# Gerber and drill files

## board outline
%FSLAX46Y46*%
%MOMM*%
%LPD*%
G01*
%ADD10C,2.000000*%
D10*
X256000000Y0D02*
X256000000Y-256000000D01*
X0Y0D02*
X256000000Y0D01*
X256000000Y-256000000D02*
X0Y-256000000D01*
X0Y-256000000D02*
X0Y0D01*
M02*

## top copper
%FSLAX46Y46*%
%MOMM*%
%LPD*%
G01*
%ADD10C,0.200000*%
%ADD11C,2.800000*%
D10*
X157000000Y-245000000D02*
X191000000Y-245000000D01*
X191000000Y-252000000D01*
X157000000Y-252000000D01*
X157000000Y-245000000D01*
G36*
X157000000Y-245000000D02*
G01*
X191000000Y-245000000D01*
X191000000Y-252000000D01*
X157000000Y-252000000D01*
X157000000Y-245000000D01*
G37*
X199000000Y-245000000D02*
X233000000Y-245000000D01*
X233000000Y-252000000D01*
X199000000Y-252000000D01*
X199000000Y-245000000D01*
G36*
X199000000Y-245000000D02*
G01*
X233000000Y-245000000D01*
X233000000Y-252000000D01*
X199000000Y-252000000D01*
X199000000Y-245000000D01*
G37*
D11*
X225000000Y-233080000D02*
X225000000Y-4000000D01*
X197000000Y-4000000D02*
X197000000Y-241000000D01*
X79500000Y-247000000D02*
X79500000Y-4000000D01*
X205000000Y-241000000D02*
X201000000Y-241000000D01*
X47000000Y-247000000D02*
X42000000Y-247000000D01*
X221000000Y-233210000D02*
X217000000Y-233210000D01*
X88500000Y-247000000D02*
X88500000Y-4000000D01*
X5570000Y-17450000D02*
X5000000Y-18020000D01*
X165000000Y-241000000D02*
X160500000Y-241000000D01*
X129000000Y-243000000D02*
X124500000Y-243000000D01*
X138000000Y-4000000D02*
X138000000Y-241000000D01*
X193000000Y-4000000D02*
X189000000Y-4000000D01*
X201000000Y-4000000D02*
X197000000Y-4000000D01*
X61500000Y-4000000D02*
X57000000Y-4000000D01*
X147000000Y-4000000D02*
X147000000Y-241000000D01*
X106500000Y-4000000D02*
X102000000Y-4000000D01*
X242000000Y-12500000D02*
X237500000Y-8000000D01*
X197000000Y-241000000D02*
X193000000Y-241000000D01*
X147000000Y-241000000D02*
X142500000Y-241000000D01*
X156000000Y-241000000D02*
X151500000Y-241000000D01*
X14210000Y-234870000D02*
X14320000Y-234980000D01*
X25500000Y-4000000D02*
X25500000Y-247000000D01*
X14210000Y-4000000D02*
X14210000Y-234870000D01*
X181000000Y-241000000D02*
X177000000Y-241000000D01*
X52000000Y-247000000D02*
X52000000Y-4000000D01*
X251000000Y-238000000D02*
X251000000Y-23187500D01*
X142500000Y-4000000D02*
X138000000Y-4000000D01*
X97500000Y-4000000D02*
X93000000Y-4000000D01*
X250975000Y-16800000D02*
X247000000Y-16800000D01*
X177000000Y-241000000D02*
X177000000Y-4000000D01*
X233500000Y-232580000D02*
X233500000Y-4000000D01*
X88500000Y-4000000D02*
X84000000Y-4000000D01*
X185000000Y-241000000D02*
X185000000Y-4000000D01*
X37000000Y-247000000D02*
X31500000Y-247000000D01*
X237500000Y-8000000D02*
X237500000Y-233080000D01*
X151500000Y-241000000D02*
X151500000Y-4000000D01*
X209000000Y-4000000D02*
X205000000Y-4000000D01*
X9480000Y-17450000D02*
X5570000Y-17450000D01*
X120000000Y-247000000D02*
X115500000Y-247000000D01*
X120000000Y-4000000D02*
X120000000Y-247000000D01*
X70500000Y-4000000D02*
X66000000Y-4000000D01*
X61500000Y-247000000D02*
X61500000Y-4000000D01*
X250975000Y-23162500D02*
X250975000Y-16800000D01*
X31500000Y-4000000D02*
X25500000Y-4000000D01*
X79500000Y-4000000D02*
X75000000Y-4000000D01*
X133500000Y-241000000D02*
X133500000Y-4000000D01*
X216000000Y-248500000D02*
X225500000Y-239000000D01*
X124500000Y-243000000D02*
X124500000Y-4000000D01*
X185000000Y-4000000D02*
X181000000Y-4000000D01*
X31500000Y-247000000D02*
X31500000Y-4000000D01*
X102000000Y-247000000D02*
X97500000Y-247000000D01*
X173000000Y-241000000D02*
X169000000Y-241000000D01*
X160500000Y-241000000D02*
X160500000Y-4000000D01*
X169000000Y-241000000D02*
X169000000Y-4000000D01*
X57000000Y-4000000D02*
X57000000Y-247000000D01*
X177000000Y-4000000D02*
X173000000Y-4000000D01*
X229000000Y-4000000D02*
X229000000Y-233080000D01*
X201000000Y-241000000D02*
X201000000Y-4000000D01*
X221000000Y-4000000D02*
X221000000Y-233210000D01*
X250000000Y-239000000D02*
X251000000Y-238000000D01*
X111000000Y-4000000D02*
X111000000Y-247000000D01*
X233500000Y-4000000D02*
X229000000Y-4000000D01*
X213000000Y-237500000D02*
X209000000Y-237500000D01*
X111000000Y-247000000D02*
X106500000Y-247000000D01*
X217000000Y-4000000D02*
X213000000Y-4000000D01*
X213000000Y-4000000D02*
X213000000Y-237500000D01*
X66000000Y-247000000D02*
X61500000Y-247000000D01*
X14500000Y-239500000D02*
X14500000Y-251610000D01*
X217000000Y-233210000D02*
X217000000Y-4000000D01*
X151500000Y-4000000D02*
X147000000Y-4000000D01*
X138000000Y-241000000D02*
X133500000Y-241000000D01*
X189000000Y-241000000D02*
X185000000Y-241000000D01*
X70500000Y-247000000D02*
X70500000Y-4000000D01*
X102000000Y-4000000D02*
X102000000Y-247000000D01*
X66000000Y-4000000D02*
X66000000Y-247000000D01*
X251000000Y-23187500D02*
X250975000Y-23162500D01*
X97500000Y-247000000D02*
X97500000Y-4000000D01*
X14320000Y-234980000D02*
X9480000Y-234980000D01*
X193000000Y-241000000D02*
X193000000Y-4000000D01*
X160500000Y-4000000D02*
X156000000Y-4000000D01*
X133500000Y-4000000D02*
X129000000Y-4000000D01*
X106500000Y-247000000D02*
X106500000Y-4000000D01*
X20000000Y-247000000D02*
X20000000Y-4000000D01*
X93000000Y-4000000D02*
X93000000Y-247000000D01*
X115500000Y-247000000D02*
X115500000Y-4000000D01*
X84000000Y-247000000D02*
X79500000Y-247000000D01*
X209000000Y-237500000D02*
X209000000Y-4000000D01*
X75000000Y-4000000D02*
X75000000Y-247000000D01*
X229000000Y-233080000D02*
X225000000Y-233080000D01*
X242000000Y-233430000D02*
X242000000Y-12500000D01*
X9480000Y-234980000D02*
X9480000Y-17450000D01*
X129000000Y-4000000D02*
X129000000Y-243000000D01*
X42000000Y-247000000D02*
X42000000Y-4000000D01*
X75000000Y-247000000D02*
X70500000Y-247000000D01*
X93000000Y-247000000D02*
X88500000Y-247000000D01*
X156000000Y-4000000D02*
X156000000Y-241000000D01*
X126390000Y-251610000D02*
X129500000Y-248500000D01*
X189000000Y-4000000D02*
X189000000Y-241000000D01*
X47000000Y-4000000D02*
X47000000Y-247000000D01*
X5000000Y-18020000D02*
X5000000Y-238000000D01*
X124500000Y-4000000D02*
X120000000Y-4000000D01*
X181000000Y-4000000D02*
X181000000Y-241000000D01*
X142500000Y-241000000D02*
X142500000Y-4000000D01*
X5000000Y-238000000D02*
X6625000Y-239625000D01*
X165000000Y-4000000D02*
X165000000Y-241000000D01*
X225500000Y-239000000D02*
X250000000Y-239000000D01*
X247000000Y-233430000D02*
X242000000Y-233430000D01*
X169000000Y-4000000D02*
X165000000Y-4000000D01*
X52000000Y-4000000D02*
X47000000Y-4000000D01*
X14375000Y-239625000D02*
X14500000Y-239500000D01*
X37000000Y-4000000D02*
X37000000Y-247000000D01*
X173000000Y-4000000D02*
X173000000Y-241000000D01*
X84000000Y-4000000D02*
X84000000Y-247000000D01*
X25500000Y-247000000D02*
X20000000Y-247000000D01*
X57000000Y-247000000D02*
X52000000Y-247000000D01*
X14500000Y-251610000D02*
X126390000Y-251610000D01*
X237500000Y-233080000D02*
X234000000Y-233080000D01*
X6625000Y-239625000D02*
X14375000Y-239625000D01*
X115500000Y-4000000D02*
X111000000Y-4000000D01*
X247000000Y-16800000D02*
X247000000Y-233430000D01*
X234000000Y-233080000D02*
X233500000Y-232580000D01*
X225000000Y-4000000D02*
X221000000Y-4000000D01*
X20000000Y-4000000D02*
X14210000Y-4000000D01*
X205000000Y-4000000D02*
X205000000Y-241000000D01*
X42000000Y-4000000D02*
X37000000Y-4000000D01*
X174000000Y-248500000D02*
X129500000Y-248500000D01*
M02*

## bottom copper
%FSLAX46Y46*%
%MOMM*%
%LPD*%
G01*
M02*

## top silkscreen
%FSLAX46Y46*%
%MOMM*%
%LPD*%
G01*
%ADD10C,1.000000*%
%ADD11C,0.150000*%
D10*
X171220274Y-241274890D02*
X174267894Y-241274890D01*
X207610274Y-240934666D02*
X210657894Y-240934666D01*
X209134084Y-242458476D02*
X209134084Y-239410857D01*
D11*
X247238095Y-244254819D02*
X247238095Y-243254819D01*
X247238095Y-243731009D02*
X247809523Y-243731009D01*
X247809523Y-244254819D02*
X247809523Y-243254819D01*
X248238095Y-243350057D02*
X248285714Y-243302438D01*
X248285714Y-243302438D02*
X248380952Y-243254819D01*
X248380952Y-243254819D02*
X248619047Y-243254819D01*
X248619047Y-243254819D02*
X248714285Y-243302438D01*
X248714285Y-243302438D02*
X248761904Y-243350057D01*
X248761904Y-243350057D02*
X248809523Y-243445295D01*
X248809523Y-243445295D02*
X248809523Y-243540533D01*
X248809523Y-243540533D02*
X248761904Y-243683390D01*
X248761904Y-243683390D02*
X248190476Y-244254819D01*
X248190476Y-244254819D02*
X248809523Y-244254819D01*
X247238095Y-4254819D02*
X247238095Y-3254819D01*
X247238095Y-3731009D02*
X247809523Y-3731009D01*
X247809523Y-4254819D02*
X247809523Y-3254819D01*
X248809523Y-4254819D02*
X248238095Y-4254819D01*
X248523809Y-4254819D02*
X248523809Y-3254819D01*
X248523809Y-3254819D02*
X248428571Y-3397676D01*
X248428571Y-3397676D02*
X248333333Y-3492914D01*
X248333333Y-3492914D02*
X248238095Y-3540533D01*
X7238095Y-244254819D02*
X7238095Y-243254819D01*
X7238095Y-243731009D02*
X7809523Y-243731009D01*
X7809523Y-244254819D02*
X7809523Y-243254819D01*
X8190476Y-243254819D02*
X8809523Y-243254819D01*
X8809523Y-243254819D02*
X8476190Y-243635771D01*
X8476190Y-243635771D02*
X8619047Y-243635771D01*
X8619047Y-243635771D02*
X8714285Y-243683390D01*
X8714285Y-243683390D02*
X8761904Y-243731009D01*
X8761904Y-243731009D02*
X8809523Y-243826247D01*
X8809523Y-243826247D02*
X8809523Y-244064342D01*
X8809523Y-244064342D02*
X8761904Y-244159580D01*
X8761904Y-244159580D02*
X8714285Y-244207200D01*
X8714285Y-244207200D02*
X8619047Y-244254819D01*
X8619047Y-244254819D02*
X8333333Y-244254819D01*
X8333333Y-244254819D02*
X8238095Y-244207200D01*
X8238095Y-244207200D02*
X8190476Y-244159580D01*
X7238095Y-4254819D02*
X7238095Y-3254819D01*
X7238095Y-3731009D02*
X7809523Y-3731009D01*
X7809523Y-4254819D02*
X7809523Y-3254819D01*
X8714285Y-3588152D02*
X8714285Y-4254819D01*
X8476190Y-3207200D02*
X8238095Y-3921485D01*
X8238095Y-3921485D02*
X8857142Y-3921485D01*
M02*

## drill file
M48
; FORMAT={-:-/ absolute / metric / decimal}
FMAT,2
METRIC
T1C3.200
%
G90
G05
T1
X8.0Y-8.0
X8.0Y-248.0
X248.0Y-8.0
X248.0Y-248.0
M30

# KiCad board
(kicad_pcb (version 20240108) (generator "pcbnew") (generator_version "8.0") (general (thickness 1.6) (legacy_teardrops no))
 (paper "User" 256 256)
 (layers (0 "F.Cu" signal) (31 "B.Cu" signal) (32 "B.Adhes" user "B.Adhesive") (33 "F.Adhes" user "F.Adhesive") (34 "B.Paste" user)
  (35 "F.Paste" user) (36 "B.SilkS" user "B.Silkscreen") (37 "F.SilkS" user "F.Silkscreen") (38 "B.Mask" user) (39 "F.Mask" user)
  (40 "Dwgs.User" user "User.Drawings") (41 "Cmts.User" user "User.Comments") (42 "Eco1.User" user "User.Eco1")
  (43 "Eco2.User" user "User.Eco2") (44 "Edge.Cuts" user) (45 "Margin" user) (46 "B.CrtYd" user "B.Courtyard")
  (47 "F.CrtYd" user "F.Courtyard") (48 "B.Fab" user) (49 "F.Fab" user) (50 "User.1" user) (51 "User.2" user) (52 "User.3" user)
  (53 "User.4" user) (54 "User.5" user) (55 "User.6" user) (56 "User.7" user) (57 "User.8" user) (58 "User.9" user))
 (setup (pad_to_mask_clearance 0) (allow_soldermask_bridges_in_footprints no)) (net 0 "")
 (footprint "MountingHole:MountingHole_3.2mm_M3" (layer "F.Cu") (at 248 248)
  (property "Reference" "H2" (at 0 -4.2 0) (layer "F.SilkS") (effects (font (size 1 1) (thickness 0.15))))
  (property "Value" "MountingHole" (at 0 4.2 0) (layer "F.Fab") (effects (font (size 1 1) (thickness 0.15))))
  (pad "" np_thru_hole circle (at 0 0) (size 3.2 3.2) (drill 3.2) (layers "*.Cu" "*.Mask")))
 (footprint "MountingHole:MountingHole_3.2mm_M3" (layer "F.Cu") (at 248 8)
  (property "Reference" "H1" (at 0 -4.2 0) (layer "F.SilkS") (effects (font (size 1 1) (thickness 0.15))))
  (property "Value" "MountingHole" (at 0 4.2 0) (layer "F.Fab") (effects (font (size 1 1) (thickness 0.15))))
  (pad "" np_thru_hole circle (at 0 0) (size 3.2 3.2) (drill 3.2) (layers "*.Cu" "*.Mask")))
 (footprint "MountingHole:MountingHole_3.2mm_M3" (layer "F.Cu") (at 8 248)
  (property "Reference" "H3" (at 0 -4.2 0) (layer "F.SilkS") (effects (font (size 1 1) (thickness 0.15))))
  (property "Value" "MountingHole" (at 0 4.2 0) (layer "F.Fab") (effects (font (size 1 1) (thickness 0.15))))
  (pad "" np_thru_hole circle (at 0 0) (size 3.2 3.2) (drill 3.2) (layers "*.Cu" "*.Mask")))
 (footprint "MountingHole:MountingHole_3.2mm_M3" (layer "F.Cu") (at 8 8)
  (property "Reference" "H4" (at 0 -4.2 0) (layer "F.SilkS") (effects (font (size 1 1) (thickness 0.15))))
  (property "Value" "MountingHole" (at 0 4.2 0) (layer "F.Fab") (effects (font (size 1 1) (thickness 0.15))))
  (pad "" np_thru_hole circle (at 0 0) (size 3.2 3.2) (drill 3.2) (layers "*.Cu" "*.Mask")))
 (gr_rect (start 157 245) (end 191 252) (stroke (width 0.2) (type solid)) (fill solid) (layer "F.Cu"))
 (gr_rect (start 199 245) (end 233 252) (stroke (width 0.2) (type solid)) (fill solid) (layer "F.Cu"))
 (gr_line (start 256 0) (end 256 256) (stroke (width 2) (type default)) (layer "Edge.Cuts"))
 (gr_line (start 0 0) (end 256 0) (stroke (width 2) (type default)) (layer "Edge.Cuts"))
 (gr_line (start 256 256) (end 0 256) (stroke (width 2) (type default)) (layer "Edge.Cuts"))
 (gr_line (start 0 256) (end 0 0) (stroke (width 2) (type default)) (layer "Edge.Cuts"))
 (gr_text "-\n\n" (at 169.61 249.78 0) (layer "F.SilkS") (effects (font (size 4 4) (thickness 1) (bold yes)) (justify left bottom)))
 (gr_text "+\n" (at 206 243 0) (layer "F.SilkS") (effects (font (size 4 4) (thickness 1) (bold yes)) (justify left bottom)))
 (segment (start 225 233.08) (end 225 4) (width 2.8) (layer "F.Cu") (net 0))
 (segment (start 197 4) (end 197 241) (width 2.8) (layer "F.Cu") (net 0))
 (segment (start 79.5 247) (end 79.5 4) (width 2.8) (layer "F.Cu") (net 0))
 (segment (start 205 241) (end 201 241) (width 2.8) (layer "F.Cu") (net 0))
 (segment (start 47 247) (end 42 247) (width 2.8) (layer "F.Cu") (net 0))
 (segment (start 221 233.21) (end 217 233.21) (width 2.8) (layer "F.Cu") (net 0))
 (segment (start 88.5 247) (end 88.5 4) (width 2.8) (layer "F.Cu") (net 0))
 (segment (start 5.57 17.45) (end 5 18.02) (width 2.8) (layer "F.Cu") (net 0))
 (segment (start 165 241) (end 160.5 241) (width 2.8) (layer "F.Cu") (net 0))
 (segment (start 129 243) (end 124.5 243) (width 2.8) (layer "F.Cu") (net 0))
 (segment (start 138 4) (end 138 241) (width 2.8) (layer "F.Cu") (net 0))
 (segment (start 193 4) (end 189 4) (width 2.8) (layer "F.Cu") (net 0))
 (segment (start 201 4) (end 197 4) (width 2.8) (layer "F.Cu") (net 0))
 (segment (start 61.5 4) (end 57 4) (width 2.8) (layer "F.Cu") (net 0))
 (segment (start 147 4) (end 147 241) (width 2.8) (layer "F.Cu") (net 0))
 (segment (start 106.5 4) (end 102 4) (width 2.8) (layer "F.Cu") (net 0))
 (segment (start 242 12.5) (end 237.5 8) (width 2.8) (layer "F.Cu") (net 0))
 (segment (start 197 241) (end 193 241) (width 2.8) (layer "F.Cu") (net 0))
 (segment (start 147 241) (end 142.5 241) (width 2.8) (layer "F.Cu") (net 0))
 (segment (start 156 241) (end 151.5 241) (width 2.8) (layer "F.Cu") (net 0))
 (segment (start 14.21 234.87) (end 14.32 234.98) (width 2.8) (layer "F.Cu") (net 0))
 (segment (start 25.5 4) (end 25.5 247) (width 2.8) (layer "F.Cu") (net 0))
 (segment (start 14.21 4) (end 14.21 234.87) (width 2.8) (layer "F.Cu") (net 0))
 (segment (start 181 241) (end 177 241) (width 2.8) (layer "F.Cu") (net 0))
 (segment (start 52 247) (end 52 4) (width 2.8) (layer "F.Cu") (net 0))
 (segment (start 251 238) (end 251 23.1875) (width 2.8) (layer "F.Cu") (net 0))
 (segment (start 142.5 4) (end 138 4) (width 2.8) (layer "F.Cu") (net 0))
 (segment (start 97.5 4) (end 93 4) (width 2.8) (layer "F.Cu") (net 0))
 (segment (start 250.975 16.8) (end 247 16.8) (width 2.8) (layer "F.Cu") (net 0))
 (segment (start 177 241) (end 177 4) (width 2.8) (layer "F.Cu") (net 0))
 (segment (start 233.5 232.58) (end 233.5 4) (width 2.8) (layer "F.Cu") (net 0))
 (segment (start 88.5 4) (end 84 4) (width 2.8) (layer "F.Cu") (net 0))
 (segment (start 185 241) (end 185 4) (width 2.8) (layer "F.Cu") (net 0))
 (segment (start 37 247) (end 31.5 247) (width 2.8) (layer "F.Cu") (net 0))
 (segment (start 237.5 8) (end 237.5 233.08) (width 2.8) (layer "F.Cu") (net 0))
 (segment (start 151.5 241) (end 151.5 4) (width 2.8) (layer "F.Cu") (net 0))
 (segment (start 209 4) (end 205 4) (width 2.8) (layer "F.Cu") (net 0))
 (segment (start 9.48 17.45) (end 5.57 17.45) (width 2.8) (layer "F.Cu") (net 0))
 (segment (start 120 247) (end 115.5 247) (width 2.8) (layer "F.Cu") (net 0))
 (segment (start 120 4) (end 120 247) (width 2.8) (layer "F.Cu") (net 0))
 (segment (start 70.5 4) (end 66 4) (width 2.8) (layer "F.Cu") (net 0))
 (segment (start 61.5 247) (end 61.5 4) (width 2.8) (layer "F.Cu") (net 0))
 (segment (start 250.975 23.1625) (end 250.975 16.8) (width 2.8) (layer "F.Cu") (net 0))
 (segment (start 31.5 4) (end 25.5 4) (width 2.8) (layer "F.Cu") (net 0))
 (segment (start 79.5 4) (end 75 4) (width 2.8) (layer "F.Cu") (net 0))
 (segment (start 133.5 241) (end 133.5 4) (width 2.8) (layer "F.Cu") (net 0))
 (segment (start 216 248.5) (end 225.5 239) (width 2.8) (layer "F.Cu") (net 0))
 (segment (start 124.5 243) (end 124.5 4) (width 2.8) (layer "F.Cu") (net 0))
 (segment (start 185 4) (end 181 4) (width 2.8) (layer "F.Cu") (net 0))
 (segment (start 31.5 247) (end 31.5 4) (width 2.8) (layer "F.Cu") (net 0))
 (segment (start 102 247) (end 97.5 247) (width 2.8) (layer "F.Cu") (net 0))
 (segment (start 173 241) (end 169 241) (width 2.8) (layer "F.Cu") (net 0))
 (segment (start 160.5 241) (end 160.5 4) (width 2.8) (layer "F.Cu") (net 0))
 (segment (start 169 241) (end 169 4) (width 2.8) (layer "F.Cu") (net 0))
 (segment (start 57 4) (end 57 247) (width 2.8) (layer "F.Cu") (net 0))
 (segment (start 177 4) (end 173 4) (width 2.8) (layer "F.Cu") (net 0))
 (segment (start 229 4) (end 229 233.08) (width 2.8) (layer "F.Cu") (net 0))
 (segment (start 201 241) (end 201 4) (width 2.8) (layer "F.Cu") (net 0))
 (segment (start 221 4) (end 221 233.21) (width 2.8) (layer "F.Cu") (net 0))
 (segment (start 250 239) (end 251 238) (width 2.8) (layer "F.Cu") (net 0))
 (segment (start 111 4) (end 111 247) (width 2.8) (layer "F.Cu") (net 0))
 (segment (start 233.5 4) (end 229 4) (width 2.8) (layer "F.Cu") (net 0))
 (segment (start 213 237.5) (end 209 237.5) (width 2.8) (layer "F.Cu") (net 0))
 (segment (start 111 247) (end 106.5 247) (width 2.8) (layer "F.Cu") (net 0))
 (segment (start 217 4) (end 213 4) (width 2.8) (layer "F.Cu") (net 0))
 (segment (start 213 4) (end 213 237.5) (width 2.8) (layer "F.Cu") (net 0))
 (segment (start 66 247) (end 61.5 247) (width 2.8) (layer "F.Cu") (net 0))
 (segment (start 14.5 239.5) (end 14.5 251.61) (width 2.8) (layer "F.Cu") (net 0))
 (segment (start 217 233.21) (end 217 4) (width 2.8) (layer "F.Cu") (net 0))
 (segment (start 151.5 4) (end 147 4) (width 2.8) (layer "F.Cu") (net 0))
 (segment (start 138 241) (end 133.5 241) (width 2.8) (layer "F.Cu") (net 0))
 (segment (start 189 241) (end 185 241) (width 2.8) (layer "F.Cu") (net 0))
 (segment (start 70.5 247) (end 70.5 4) (width 2.8) (layer "F.Cu") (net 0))
 (segment (start 102 4) (end 102 247) (width 2.8) (layer "F.Cu") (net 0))
 (segment (start 66 4) (end 66 247) (width 2.8) (layer "F.Cu") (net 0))
 (segment (start 251 23.1875) (end 250.975 23.1625) (width 2.8) (layer "F.Cu") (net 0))
 (segment (start 97.5 247) (end 97.5 4) (width 2.8) (layer "F.Cu") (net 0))
 (segment (start 14.32 234.98) (end 9.48 234.98) (width 2.8) (layer "F.Cu") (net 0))
 (segment (start 193 241) (end 193 4) (width 2.8) (layer "F.Cu") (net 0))
 (segment (start 160.5 4) (end 156 4) (width 2.8) (layer "F.Cu") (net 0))
 (segment (start 133.5 4) (end 129 4) (width 2.8) (layer "F.Cu") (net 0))
 (segment (start 106.5 247) (end 106.5 4) (width 2.8) (layer "F.Cu") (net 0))
 (segment (start 20 247) (end 20 4) (width 2.8) (layer "F.Cu") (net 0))
 (segment (start 93 4) (end 93 247) (width 2.8) (layer "F.Cu") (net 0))
 (segment (start 115.5 247) (end 115.5 4) (width 2.8) (layer "F.Cu") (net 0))
 (segment (start 84 247) (end 79.5 247) (width 2.8) (layer "F.Cu") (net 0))
 (segment (start 209 237.5) (end 209 4) (width 2.8) (layer "F.Cu") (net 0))
 (segment (start 75 4) (end 75 247) (width 2.8) (layer "F.Cu") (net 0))
 (segment (start 229 233.08) (end 225 233.08) (width 2.8) (layer "F.Cu") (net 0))
 (segment (start 242 233.43) (end 242 12.5) (width 2.8) (layer "F.Cu") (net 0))
 (segment (start 9.48 234.98) (end 9.48 17.45) (width 2.8) (layer "F.Cu") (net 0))
 (segment (start 129 4) (end 129 243) (width 2.8) (layer "F.Cu") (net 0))
 (segment (start 42 247) (end 42 4) (width 2.8) (layer "F.Cu") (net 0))
 (segment (start 75 247) (end 70.5 247) (width 2.8) (layer "F.Cu") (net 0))
 (segment (start 93 247) (end 88.5 247) (width 2.8) (layer "F.Cu") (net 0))
 (segment (start 156 4) (end 156 241) (width 2.8) (layer "F.Cu") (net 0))
 (segment (start 126.39 251.61) (end 129.5 248.5) (width 2.8) (layer "F.Cu") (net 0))
 (segment (start 189 4) (end 189 241) (width 2.8) (layer "F.Cu") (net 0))
 (segment (start 47 4) (end 47 247) (width 2.8) (layer "F.Cu") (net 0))
 (segment (start 5 18.02) (end 5 238) (width 2.8) (layer "F.Cu") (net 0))
 (segment (start 124.5 4) (end 120 4) (width 2.8) (layer "F.Cu") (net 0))
 (segment (start 181 4) (end 181 241) (width 2.8) (layer "F.Cu") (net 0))
 (segment (start 142.5 241) (end 142.5 4) (width 2.8) (layer "F.Cu") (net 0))
 (segment (start 5 238) (end 6.625 239.625) (width 2.8) (layer "F.Cu") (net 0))
 (segment (start 165 4) (end 165 241) (width 2.8) (layer "F.Cu") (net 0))
 (segment (start 225.5 239) (end 250 239) (width 2.8) (layer "F.Cu") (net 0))
 (segment (start 247 233.43) (end 242 233.43) (width 2.8) (layer "F.Cu") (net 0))
 (segment (start 169 4) (end 165 4) (width 2.8) (layer "F.Cu") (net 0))
 (segment (start 52 4) (end 47 4) (width 2.8) (layer "F.Cu") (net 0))
 (segment (start 14.375 239.625) (end 14.5 239.5) (width 2.8) (layer "F.Cu") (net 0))
 (segment (start 37 4) (end 37 247) (width 2.8) (layer "F.Cu") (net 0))
 (segment (start 173 4) (end 173 241) (width 2.8) (layer "F.Cu") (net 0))
 (segment (start 84 4) (end 84 247) (width 2.8) (layer "F.Cu") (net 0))
 (segment (start 25.5 247) (end 20 247) (width 2.8) (layer "F.Cu") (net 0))
 (segment (start 57 247) (end 52 247) (width 2.8) (layer "F.Cu") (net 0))
 (segment (start 14.5 251.61) (end 126.39 251.61) (width 2.8) (layer "F.Cu") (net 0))
 (segment (start 237.5 233.08) (end 234 233.08) (width 2.8) (layer "F.Cu") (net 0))
 (segment (start 6.625 239.625) (end 14.375 239.625) (width 2.8) (layer "F.Cu") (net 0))
 (segment (start 115.5 4) (end 111 4) (width 2.8) (layer "F.Cu") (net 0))
 (segment (start 247 16.8) (end 247 233.43) (width 2.8) (layer "F.Cu") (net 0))
 (segment (start 234 233.08) (end 233.5 232.58) (width 2.8) (layer "F.Cu") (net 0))
 (segment (start 225 4) (end 221 4) (width 2.8) (layer "F.Cu") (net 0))
 (segment (start 20 4) (end 14.21 4) (width 2.8) (layer "F.Cu") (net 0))
 (segment (start 205 4) (end 205 241) (width 2.8) (layer "F.Cu") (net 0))
 (segment (start 42 4) (end 37 4) (width 2.8) (layer "F.Cu") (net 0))
 (segment (start 174 248.5) (end 129.5 248.5) (width 2.8) (layer "F.Cu") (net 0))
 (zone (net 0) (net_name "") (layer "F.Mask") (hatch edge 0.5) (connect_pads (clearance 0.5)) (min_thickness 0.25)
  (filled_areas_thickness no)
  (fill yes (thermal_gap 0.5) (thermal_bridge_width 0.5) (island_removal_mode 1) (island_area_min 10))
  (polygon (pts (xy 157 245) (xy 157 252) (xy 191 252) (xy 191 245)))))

